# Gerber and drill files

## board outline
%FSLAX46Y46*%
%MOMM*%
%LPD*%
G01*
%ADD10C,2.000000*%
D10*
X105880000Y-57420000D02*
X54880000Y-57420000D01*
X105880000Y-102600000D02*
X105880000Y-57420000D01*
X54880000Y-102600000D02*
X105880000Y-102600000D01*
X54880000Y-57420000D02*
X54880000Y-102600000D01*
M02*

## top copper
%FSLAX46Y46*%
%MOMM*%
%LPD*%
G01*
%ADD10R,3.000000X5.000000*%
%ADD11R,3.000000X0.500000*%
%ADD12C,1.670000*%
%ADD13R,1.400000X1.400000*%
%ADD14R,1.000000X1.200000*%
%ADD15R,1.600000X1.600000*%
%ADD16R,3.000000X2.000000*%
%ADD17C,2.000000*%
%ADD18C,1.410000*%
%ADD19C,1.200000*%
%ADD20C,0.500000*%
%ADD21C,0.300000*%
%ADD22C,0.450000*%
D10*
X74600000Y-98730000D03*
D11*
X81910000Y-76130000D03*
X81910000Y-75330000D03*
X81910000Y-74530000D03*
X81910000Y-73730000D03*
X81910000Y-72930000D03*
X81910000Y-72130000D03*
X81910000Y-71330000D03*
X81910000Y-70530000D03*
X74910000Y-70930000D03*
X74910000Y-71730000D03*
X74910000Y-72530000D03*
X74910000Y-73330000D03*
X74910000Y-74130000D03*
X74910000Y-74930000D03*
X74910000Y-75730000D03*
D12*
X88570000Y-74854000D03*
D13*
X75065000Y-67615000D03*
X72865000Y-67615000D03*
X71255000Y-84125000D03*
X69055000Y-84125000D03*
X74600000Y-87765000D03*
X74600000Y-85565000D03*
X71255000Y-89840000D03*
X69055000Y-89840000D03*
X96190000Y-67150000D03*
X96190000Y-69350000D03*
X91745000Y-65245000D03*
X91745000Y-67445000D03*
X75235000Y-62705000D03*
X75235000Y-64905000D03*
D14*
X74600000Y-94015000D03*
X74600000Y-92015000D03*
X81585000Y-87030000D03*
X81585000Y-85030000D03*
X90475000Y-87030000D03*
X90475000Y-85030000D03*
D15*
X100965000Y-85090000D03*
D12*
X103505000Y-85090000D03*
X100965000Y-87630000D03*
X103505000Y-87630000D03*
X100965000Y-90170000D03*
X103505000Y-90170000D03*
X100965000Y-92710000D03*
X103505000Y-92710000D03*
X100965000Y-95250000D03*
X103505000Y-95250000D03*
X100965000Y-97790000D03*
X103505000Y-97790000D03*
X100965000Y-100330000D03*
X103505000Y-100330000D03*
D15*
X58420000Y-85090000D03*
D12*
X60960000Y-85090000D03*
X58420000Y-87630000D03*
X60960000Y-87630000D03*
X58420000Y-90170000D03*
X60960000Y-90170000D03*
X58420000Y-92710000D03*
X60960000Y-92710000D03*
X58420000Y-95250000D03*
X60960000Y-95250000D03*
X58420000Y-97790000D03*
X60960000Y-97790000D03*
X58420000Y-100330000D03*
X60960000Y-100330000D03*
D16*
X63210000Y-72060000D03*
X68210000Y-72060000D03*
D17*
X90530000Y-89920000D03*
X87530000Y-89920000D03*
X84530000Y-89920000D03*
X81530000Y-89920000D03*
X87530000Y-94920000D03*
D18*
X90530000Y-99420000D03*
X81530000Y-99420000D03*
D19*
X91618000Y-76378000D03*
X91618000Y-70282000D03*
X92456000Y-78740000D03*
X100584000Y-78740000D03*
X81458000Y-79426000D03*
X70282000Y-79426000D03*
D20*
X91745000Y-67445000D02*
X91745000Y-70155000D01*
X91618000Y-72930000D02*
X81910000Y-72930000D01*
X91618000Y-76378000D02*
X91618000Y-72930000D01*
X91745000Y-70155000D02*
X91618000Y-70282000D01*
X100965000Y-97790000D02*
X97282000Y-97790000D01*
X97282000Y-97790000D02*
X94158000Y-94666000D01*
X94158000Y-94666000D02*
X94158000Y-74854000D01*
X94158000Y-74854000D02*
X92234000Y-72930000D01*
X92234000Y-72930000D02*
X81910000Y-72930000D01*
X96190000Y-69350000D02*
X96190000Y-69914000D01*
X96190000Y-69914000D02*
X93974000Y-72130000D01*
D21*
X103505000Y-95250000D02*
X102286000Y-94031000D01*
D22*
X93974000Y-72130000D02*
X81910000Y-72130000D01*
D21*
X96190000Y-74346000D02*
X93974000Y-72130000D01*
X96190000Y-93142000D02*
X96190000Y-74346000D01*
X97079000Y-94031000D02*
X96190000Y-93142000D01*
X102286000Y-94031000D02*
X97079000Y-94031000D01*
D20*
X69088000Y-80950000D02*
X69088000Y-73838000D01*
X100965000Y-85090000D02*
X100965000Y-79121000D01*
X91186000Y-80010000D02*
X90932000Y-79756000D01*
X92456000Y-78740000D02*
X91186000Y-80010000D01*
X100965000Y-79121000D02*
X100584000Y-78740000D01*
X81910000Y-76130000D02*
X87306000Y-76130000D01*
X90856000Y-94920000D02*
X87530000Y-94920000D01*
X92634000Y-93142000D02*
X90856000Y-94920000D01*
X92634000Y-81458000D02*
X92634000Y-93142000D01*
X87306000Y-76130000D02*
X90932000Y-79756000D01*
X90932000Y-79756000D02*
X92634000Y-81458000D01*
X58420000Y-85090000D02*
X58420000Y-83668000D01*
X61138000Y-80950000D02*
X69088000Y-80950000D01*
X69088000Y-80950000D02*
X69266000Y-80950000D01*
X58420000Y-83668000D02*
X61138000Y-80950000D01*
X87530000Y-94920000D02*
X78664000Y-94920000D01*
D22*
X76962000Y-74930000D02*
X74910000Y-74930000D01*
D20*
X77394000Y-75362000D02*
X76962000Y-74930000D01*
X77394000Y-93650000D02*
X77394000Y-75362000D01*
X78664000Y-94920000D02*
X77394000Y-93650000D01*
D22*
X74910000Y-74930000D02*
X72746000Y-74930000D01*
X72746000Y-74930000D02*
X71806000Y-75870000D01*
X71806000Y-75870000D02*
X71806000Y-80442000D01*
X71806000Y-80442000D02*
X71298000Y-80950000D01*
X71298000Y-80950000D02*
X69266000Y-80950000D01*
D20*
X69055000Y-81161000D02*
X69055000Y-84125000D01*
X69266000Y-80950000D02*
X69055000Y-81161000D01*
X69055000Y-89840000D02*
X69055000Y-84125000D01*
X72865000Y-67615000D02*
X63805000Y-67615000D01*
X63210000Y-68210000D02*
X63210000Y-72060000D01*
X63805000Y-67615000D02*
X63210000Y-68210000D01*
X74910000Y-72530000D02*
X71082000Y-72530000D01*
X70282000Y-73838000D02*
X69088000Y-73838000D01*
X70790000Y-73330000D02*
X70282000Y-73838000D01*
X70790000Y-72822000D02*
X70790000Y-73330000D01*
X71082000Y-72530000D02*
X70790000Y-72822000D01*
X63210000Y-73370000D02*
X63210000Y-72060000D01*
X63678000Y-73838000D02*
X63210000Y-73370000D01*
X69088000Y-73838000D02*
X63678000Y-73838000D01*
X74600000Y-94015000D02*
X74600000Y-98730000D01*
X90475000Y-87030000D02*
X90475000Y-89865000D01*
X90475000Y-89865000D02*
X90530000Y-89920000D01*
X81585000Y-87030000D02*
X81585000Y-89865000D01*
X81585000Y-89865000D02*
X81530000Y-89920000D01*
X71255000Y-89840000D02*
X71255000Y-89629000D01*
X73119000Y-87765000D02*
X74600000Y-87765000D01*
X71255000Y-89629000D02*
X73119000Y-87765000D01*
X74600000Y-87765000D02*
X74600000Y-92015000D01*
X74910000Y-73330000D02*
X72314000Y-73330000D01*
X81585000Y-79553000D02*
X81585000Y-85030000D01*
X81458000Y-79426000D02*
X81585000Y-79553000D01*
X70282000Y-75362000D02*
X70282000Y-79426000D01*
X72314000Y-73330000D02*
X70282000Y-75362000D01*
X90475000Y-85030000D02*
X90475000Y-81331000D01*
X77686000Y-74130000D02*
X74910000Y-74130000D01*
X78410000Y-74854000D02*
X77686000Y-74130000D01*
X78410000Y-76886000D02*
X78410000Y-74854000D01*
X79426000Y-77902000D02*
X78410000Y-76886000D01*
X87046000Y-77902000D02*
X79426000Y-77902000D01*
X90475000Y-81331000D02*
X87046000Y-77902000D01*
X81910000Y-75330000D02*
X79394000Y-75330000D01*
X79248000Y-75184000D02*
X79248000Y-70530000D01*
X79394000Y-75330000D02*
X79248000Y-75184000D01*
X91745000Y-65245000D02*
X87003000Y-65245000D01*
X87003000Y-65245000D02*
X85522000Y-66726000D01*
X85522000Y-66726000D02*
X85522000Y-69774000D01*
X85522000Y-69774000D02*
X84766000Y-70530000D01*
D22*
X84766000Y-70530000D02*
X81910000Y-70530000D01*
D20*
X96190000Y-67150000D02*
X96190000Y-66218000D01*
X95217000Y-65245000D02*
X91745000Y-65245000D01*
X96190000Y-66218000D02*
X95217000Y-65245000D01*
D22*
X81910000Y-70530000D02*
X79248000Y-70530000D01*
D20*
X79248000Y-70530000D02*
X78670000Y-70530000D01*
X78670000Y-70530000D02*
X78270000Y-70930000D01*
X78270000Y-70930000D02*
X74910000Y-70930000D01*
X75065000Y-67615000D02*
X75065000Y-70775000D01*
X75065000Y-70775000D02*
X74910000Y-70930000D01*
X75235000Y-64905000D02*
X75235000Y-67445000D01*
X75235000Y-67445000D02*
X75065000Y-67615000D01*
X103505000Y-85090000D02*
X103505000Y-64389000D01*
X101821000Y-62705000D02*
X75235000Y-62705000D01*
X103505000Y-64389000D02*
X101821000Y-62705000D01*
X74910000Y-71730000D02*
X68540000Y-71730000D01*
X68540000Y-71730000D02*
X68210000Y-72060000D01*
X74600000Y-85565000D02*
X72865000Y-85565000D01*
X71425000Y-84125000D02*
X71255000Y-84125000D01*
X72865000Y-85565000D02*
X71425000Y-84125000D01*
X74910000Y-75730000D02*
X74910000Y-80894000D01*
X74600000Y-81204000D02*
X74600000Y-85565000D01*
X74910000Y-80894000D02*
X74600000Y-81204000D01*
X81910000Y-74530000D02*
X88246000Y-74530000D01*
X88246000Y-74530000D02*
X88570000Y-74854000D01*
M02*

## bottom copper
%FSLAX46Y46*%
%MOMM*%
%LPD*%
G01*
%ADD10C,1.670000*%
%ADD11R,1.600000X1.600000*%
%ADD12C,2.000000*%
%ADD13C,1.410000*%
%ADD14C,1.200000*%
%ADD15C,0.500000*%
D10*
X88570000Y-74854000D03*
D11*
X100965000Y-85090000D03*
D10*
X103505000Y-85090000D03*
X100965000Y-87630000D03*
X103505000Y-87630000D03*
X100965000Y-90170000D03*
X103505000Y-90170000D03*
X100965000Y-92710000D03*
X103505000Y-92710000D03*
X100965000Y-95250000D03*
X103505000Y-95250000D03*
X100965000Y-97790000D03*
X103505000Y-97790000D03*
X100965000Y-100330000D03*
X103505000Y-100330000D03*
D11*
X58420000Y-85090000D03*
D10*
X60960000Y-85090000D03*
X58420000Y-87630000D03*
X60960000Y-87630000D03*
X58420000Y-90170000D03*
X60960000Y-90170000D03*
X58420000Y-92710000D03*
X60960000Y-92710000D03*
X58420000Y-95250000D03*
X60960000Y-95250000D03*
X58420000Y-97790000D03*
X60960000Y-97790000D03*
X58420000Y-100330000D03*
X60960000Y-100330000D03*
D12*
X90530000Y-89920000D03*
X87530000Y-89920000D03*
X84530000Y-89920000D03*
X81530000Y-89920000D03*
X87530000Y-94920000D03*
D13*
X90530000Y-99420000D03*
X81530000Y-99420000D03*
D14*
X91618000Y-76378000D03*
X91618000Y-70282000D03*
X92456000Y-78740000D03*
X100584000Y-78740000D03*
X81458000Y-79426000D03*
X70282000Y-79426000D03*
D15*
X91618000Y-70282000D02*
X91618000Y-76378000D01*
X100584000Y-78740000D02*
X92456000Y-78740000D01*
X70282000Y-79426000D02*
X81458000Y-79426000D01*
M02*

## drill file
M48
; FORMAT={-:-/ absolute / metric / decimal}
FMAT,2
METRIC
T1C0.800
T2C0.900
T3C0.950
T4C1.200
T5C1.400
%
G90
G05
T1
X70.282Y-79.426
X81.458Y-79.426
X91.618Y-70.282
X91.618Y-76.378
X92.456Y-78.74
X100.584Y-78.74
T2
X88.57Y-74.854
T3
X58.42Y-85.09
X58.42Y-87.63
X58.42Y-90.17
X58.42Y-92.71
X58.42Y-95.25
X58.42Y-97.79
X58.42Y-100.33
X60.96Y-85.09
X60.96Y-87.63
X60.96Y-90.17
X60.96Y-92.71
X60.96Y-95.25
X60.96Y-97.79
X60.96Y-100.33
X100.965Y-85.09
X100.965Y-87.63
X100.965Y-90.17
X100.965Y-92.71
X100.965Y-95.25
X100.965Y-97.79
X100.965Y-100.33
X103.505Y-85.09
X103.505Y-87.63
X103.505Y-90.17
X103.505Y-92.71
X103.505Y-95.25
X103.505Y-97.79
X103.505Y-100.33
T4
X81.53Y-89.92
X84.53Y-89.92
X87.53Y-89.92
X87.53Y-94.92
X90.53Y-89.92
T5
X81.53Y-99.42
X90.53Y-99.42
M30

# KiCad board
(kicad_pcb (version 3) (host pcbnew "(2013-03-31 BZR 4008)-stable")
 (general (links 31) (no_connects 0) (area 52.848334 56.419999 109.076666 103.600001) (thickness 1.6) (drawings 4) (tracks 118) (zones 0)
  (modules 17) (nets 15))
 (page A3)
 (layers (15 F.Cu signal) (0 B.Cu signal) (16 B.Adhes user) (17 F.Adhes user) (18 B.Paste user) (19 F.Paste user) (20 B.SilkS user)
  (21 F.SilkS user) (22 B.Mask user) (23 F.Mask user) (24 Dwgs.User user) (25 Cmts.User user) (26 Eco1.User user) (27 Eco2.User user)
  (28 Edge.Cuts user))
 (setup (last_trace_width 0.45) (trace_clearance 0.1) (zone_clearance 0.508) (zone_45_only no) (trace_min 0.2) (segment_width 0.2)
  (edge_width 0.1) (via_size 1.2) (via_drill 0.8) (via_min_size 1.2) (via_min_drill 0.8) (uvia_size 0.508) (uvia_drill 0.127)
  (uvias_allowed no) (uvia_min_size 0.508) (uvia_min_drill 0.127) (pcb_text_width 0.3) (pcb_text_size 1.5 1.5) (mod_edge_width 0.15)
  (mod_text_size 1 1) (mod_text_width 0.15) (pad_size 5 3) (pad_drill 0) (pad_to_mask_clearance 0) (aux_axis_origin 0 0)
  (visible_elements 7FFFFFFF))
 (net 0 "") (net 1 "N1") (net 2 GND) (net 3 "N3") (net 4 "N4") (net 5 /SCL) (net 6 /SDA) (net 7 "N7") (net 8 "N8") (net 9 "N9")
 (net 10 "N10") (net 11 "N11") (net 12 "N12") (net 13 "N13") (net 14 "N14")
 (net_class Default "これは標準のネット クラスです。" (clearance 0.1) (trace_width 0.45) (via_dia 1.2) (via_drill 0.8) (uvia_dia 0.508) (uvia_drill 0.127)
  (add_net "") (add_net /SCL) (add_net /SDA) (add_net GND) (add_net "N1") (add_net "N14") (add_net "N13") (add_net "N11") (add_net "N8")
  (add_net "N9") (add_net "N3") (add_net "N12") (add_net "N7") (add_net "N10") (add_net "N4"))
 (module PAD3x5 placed (layer F.Cu) (at 74.6 98.73 90)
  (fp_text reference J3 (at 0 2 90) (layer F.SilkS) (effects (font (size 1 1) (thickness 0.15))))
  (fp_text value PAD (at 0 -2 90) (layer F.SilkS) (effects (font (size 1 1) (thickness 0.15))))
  (pad 1 smd rect (at 0 0 90) (size 5 3) (layers F.Cu F.Paste F.Mask) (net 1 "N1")))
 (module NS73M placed (layer F.Cu) (at 78.41 73.33)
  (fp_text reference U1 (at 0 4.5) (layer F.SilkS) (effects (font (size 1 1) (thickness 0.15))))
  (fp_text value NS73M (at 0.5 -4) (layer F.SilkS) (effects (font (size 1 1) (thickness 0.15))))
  (pad 1 smd rect (at 3.5 2.8) (size 3 0.5) (layers F.Cu F.Paste F.Mask) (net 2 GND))
  (pad 2 smd rect (at 3.5 2) (size 3 0.5) (layers F.Cu F.Paste F.Mask) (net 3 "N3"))
  (pad 3 smd rect (at 3.5 1.2) (size 3 0.5) (layers F.Cu F.Paste F.Mask) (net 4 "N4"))
  (pad 4 smd rect (at 3.5 0.4) (size 3 0.5) (layers F.Cu F.Paste F.Mask))
  (pad 5 smd rect (at 3.5 -0.4) (size 3 0.5) (layers F.Cu F.Paste F.Mask) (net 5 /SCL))
  (pad 6 smd rect (at 3.5 -1.2) (size 3 0.5) (layers F.Cu F.Paste F.Mask) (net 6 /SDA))
  (pad 7 smd rect (at 3.5 -2) (size 3 0.5) (layers F.Cu F.Paste F.Mask))
  (pad 8 smd rect (at 3.5 -2.8) (size 3 0.5) (layers F.Cu F.Paste F.Mask) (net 3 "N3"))
  (pad 9 smd rect (at -3.5 -2.4) (size 3 0.5) (layers F.Cu F.Paste F.Mask) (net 3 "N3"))
  (pad 10 smd rect (at -3.5 -1.6) (size 3 0.5) (layers F.Cu F.Paste F.Mask) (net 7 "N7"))
  (pad 11 smd rect (at -3.5 -0.8) (size 3 0.5) (layers F.Cu F.Paste F.Mask) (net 2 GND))
  (pad 12 smd rect (at -3.5 0) (size 3 0.5) (layers F.Cu F.Paste F.Mask) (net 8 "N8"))
  (pad 13 smd rect (at -3.5 0.8) (size 3 0.5) (layers F.Cu F.Paste F.Mask) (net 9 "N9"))
  (pad 14 smd rect (at -3.5 1.6) (size 3 0.5) (layers F.Cu F.Paste F.Mask) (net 2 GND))
  (pad 15 smd rect (at -3.5 2.4) (size 3 0.5) (layers F.Cu F.Paste F.Mask) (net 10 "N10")))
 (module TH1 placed (layer F.Cu) (at 88.57 74.854)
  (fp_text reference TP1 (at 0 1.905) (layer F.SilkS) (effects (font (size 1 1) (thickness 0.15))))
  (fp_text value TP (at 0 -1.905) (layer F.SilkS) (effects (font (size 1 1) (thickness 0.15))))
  (pad 1 thru_hole circle (at 0 0) (size 1.67 1.67) (drill 0.9) (layers *.Cu *.Mask F.SilkS) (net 4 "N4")))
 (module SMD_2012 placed (layer F.Cu) (at 73.965 67.615 180)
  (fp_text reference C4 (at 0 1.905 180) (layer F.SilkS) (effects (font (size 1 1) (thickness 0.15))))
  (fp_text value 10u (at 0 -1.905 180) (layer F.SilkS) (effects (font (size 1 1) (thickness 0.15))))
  (pad 1 smd rect (at -1.1 0 180) (size 1.4 1.4) (layers F.Cu F.Paste F.Mask) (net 3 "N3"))
  (pad 2 smd rect (at 1.1 0 180) (size 1.4 1.4) (layers F.Cu F.Paste F.Mask) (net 2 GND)))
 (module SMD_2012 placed (layer F.Cu) (at 70.155 84.125 180)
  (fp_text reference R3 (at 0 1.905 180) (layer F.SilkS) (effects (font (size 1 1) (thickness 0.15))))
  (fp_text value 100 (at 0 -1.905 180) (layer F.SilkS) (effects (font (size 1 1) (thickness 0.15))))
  (pad 1 smd rect (at -1.1 0 180) (size 1.4 1.4) (layers F.Cu F.Paste F.Mask) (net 10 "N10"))
  (pad 2 smd rect (at 1.1 0 180) (size 1.4 1.4) (layers F.Cu F.Paste F.Mask) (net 2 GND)))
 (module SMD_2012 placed (layer F.Cu) (at 74.6 86.665 90)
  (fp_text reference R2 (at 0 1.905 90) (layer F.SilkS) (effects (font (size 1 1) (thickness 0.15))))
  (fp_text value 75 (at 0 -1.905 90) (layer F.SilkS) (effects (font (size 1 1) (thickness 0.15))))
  (pad 1 smd rect (at -1.1 0 90) (size 1.4 1.4) (layers F.Cu F.Paste F.Mask) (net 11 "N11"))
  (pad 2 smd rect (at 1.1 0 90) (size 1.4 1.4) (layers F.Cu F.Paste F.Mask) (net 10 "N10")))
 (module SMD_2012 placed (layer F.Cu) (at 70.155 89.84 180)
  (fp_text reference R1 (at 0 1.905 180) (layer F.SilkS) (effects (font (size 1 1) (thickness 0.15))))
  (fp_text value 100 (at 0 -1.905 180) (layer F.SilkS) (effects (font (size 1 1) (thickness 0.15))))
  (pad 1 smd rect (at -1.1 0 180) (size 1.4 1.4) (layers F.Cu F.Paste F.Mask) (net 11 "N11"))
  (pad 2 smd rect (at 1.1 0 180) (size 1.4 1.4) (layers F.Cu F.Paste F.Mask) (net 2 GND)))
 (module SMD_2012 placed (layer F.Cu) (at 96.19 68.25 270)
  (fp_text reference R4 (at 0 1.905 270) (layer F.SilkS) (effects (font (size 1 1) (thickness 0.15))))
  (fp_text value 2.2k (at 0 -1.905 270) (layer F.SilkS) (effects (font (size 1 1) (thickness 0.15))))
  (pad 1 smd rect (at -1.1 0 270) (size 1.4 1.4) (layers F.Cu F.Paste F.Mask) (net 3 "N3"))
  (pad 2 smd rect (at 1.1 0 270) (size 1.4 1.4) (layers F.Cu F.Paste F.Mask) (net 6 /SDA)))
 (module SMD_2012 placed (layer F.Cu) (at 91.745 66.345 270)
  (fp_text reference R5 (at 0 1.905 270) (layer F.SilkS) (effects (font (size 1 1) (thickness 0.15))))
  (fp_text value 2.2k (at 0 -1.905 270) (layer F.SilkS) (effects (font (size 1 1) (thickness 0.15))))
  (pad 1 smd rect (at -1.1 0 270) (size 1.4 1.4) (layers F.Cu F.Paste F.Mask) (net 3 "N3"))
  (pad 2 smd rect (at 1.1 0 270) (size 1.4 1.4) (layers F.Cu F.Paste F.Mask) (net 5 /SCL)))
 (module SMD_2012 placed (layer F.Cu) (at 75.235 63.805 270)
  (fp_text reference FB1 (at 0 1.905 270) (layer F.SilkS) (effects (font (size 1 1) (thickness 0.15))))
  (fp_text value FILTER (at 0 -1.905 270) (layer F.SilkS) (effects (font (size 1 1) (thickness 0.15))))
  (pad 1 smd rect (at -1.1 0 270) (size 1.4 1.4) (layers F.Cu F.Paste F.Mask) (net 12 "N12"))
  (pad 2 smd rect (at 1.1 0 270) (size 1.4 1.4) (layers F.Cu F.Paste F.Mask) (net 3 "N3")))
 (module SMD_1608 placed (layer F.Cu) (at 74.6 93.015 90)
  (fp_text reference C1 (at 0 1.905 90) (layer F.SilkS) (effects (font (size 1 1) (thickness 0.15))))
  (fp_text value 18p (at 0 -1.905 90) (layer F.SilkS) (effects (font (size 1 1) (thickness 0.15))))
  (pad 1 smd rect (at -1 0 90) (size 1.2 1) (layers F.Cu F.Paste F.Mask) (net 1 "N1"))
  (pad 2 smd rect (at 1 0 90) (size 1.2 1) (layers F.Cu F.Paste F.Mask) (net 11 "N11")))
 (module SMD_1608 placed (layer F.Cu) (at 81.585 86.03 90)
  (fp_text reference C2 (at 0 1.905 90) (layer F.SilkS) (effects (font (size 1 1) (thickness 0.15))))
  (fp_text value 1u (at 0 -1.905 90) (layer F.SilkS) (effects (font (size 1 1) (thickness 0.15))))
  (pad 1 smd rect (at -1 0 90) (size 1.2 1) (layers F.Cu F.Paste F.Mask) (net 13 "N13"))
  (pad 2 smd rect (at 1 0 90) (size 1.2 1) (layers F.Cu F.Paste F.Mask) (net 8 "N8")))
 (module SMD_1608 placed (layer F.Cu) (at 90.475 86.03 90)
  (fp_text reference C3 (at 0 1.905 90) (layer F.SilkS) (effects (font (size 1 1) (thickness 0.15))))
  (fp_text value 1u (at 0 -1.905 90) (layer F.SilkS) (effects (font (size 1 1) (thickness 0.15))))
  (pad 1 smd rect (at -1 0 90) (size 1.2 1) (layers F.Cu F.Paste F.Mask) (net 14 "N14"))
  (pad 2 smd rect (at 1 0 90) (size 1.2 1) (layers F.Cu F.Paste F.Mask) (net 9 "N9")))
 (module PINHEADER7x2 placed (layer F.Cu) (at 102.235 92.71)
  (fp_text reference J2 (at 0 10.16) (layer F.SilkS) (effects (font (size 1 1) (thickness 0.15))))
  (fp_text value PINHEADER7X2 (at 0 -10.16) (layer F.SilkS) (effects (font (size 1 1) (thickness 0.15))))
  (pad 1 thru_hole rect (at -1.27 -7.62) (size 1.6 1.6) (drill 0.95) (layers *.Cu *.Mask F.SilkS) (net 2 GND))
  (pad 2 thru_hole circle (at 1.27 -7.62) (size 1.67 1.67) (drill 0.95) (layers *.Cu *.Mask F.SilkS) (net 12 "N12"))
  (pad 3 thru_hole circle (at -1.27 -5.08) (size 1.67 1.67) (drill 0.95) (layers *.Cu *.Mask F.SilkS))
  (pad 4 thru_hole circle (at 1.27 -5.08) (size 1.67 1.67) (drill 0.95) (layers *.Cu *.Mask F.SilkS))
  (pad 5 thru_hole circle (at -1.27 -2.54) (size 1.67 1.67) (drill 0.95) (layers *.Cu *.Mask F.SilkS))
  (pad 6 thru_hole circle (at 1.27 -2.54) (size 1.67 1.67) (drill 0.95) (layers *.Cu *.Mask F.SilkS))
  (pad 7 thru_hole circle (at -1.27 0) (size 1.67 1.67) (drill 0.95) (layers *.Cu *.Mask F.SilkS))
  (pad 8 thru_hole circle (at 1.27 0) (size 1.67 1.67) (drill 0.95) (layers *.Cu *.Mask F.SilkS))
  (pad 9 thru_hole circle (at -1.27 2.54) (size 1.67 1.67) (drill 0.95) (layers *.Cu *.Mask F.SilkS))
  (pad 10 thru_hole circle (at 1.27 2.54) (size 1.67 1.67) (drill 0.95) (layers *.Cu *.Mask F.SilkS) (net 6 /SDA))
  (pad 11 thru_hole circle (at -1.27 5.08) (size 1.67 1.67) (drill 0.95) (layers *.Cu *.Mask F.SilkS) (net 5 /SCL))
  (pad 12 thru_hole circle (at 1.27 5.08) (size 1.67 1.67) (drill 0.95) (layers *.Cu *.Mask F.SilkS))
  (pad 13 thru_hole circle (at -1.27 7.62) (size 1.67 1.67) (drill 0.95) (layers *.Cu *.Mask F.SilkS))
  (pad 14 thru_hole circle (at 1.27 7.62) (size 1.67 1.67) (drill 0.95) (layers *.Cu *.Mask F.SilkS)))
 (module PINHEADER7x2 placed (layer F.Cu) (at 59.69 92.71)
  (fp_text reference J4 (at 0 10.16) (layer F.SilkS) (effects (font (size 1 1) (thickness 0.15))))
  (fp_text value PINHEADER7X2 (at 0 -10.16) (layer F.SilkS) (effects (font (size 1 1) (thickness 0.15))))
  (pad 1 thru_hole rect (at -1.27 -7.62) (size 1.6 1.6) (drill 0.95) (layers *.Cu *.Mask F.SilkS) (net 2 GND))
  (pad 2 thru_hole circle (at 1.27 -7.62) (size 1.67 1.67) (drill 0.95) (layers *.Cu *.Mask F.SilkS))
  (pad 3 thru_hole circle (at -1.27 -5.08) (size 1.67 1.67) (drill 0.95) (layers *.Cu *.Mask F.SilkS))
  (pad 4 thru_hole circle (at 1.27 -5.08) (size 1.67 1.67) (drill 0.95) (layers *.Cu *.Mask F.SilkS))
  (pad 5 thru_hole circle (at -1.27 -2.54) (size 1.67 1.67) (drill 0.95) (layers *.Cu *.Mask F.SilkS))
  (pad 6 thru_hole circle (at 1.27 -2.54) (size 1.67 1.67) (drill 0.95) (layers *.Cu *.Mask F.SilkS))
  (pad 7 thru_hole circle (at -1.27 0) (size 1.67 1.67) (drill 0.95) (layers *.Cu *.Mask F.SilkS))
  (pad 8 thru_hole circle (at 1.27 0) (size 1.67 1.67) (drill 0.95) (layers *.Cu *.Mask F.SilkS))
  (pad 9 thru_hole circle (at -1.27 2.54) (size 1.67 1.67) (drill 0.95) (layers *.Cu *.Mask F.SilkS))
  (pad 10 thru_hole circle (at 1.27 2.54) (size 1.67 1.67) (drill 0.95) (layers *.Cu *.Mask F.SilkS))
  (pad 11 thru_hole circle (at -1.27 5.08) (size 1.67 1.67) (drill 0.95) (layers *.Cu *.Mask F.SilkS))
  (pad 12 thru_hole circle (at 1.27 5.08) (size 1.67 1.67) (drill 0.95) (layers *.Cu *.Mask F.SilkS))
  (pad 13 thru_hole circle (at -1.27 7.62) (size 1.67 1.67) (drill 0.95) (layers *.Cu *.Mask F.SilkS))
  (pad 14 thru_hole circle (at 1.27 7.62) (size 1.67 1.67) (drill 0.95) (layers *.Cu *.Mask F.SilkS)))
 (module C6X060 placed (layer F.Cu) (at 65.71 72.06)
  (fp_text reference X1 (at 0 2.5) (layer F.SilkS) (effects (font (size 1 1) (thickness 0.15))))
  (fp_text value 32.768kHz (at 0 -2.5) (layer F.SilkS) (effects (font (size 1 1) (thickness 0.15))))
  (pad 1 smd rect (at -2.5 0) (size 3 2) (layers F.Cu F.Paste F.Mask) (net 2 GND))
  (pad 2 smd rect (at 2.5 0) (size 3 2) (layers F.Cu F.Paste F.Mask) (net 7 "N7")))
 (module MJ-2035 (layer B.Cu) (at 86.03 94.92 180)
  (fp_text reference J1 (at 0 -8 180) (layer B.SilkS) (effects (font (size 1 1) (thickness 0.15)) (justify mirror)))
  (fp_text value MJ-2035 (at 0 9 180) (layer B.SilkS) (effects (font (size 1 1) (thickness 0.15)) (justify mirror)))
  (pad 1 thru_hole circle (at -4.5 5 180) (size 2 2) (drill 1.2) (layers *.Cu *.Mask B.SilkS) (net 14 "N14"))
  (pad 2 thru_hole circle (at -1.5 5 180) (size 2 2) (drill 1.2) (layers *.Cu *.Mask B.SilkS))
  (pad 3 thru_hole circle (at 1.5 5 180) (size 2 2) (drill 1.2) (layers *.Cu *.Mask B.SilkS))
  (pad 4 thru_hole circle (at 4.5 5 180) (size 2 2) (drill 1.2) (layers *.Cu *.Mask B.SilkS) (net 13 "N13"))
  (pad 5 thru_hole circle (at -1.5 0 180) (size 2 2) (drill 1.2) (layers *.Cu *.Mask B.SilkS) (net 2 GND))
  (pad "" thru_hole circle (at -4.5 -4.5 180) (size 1.41 1.41) (drill 1.4) (layers *.Cu *.Mask B.SilkS))
  (pad "" thru_hole circle (at 4.5 -4.5 180) (size 1.41 1.41) (drill 1.4) (layers *.Cu *.Mask B.SilkS)))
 (gr_line (start 105.88 57.42) (end 54.88 57.42) (angle 90) (layer Edge.Cuts) (width 2))
 (gr_line (start 105.88 102.6) (end 105.88 57.42) (angle 90) (layer Edge.Cuts) (width 2))
 (gr_line (start 54.88 102.6) (end 105.88 102.6) (angle 90) (layer Edge.Cuts) (width 2))
 (gr_line (start 54.88 57.42) (end 54.88 102.6) (angle 90) (layer Edge.Cuts) (width 2))
 (segment (start 91.745 67.445) (end 91.745 70.155) (width 0.5) (layer F.Cu) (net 5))
 (segment (start 91.618 72.93) (end 81.91 72.93) (width 0.5) (layer F.Cu) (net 5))
 (segment (start 91.618 76.378) (end 91.618 72.93) (width 0.5) (layer F.Cu) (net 5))
 (via (at 91.618 76.378) (size 1.2) (layers F.Cu B.Cu) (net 5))
 (segment (start 91.618 70.282) (end 91.618 76.378) (width 0.5) (layer B.Cu) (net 5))
 (via (at 91.618 70.282) (size 1.2) (layers F.Cu B.Cu) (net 5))
 (segment (start 91.745 70.155) (end 91.618 70.282) (width 0.5) (layer F.Cu) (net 5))
 (segment (start 100.965 97.79) (end 97.282 97.79) (width 0.5) (layer F.Cu) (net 5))
 (segment (start 97.282 97.79) (end 94.158 94.666) (width 0.5) (layer F.Cu) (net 5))
 (segment (start 94.158 94.666) (end 94.158 74.854) (width 0.5) (layer F.Cu) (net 5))
 (segment (start 94.158 74.854) (end 92.234 72.93) (width 0.5) (layer F.Cu) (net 5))
 (segment (start 92.234 72.93) (end 81.91 72.93) (width 0.5) (layer F.Cu) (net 5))
 (segment (start 96.19 69.35) (end 96.19 69.914) (width 0.5) (layer F.Cu) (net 6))
 (segment (start 96.19 69.914) (end 93.974 72.13) (width 0.5) (layer F.Cu) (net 6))
 (segment (start 103.505 95.25) (end 102.286 94.031) (width 0.3) (layer F.Cu) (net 6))
 (segment (start 93.974 72.13) (end 81.91 72.13) (width 0.45) (layer F.Cu) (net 6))
 (segment (start 96.19 74.346) (end 93.974 72.13) (width 0.3) (layer F.Cu) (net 6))
 (segment (start 96.19 93.142) (end 96.19 74.346) (width 0.3) (layer F.Cu) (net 6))
 (segment (start 97.079 94.031) (end 96.19 93.142) (width 0.3) (layer F.Cu) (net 6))
 (segment (start 102.286 94.031) (end 97.079 94.031) (width 0.3) (layer F.Cu) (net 6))
 (segment (start 69.088 80.95) (end 69.088 73.838) (width 0.5) (layer F.Cu) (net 2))
 (segment (start 100.965 85.09) (end 100.965 79.121) (width 0.5) (layer F.Cu) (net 2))
 (segment (start 91.186 80.01) (end 90.932 79.756) (width 0.5) (layer F.Cu) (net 2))
 (segment (start 92.456 78.74) (end 91.186 80.01) (width 0.5) (layer F.Cu) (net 2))
 (via (at 92.456 78.74) (size 1.2) (layers F.Cu B.Cu) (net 2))
 (segment (start 100.584 78.74) (end 92.456 78.74) (width 0.5) (layer B.Cu) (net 2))
 (via (at 100.584 78.74) (size 1.2) (layers F.Cu B.Cu) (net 2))
 (segment (start 100.965 79.121) (end 100.584 78.74) (width 0.5) (layer F.Cu) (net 2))
 (segment (start 81.91 76.13) (end 87.306 76.13) (width 0.5) (layer F.Cu) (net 2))
 (segment (start 90.856 94.92) (end 87.53 94.92) (width 0.5) (layer F.Cu) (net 2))
 (segment (start 92.634 93.142) (end 90.856 94.92) (width 0.5) (layer F.Cu) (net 2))
 (segment (start 92.634 81.458) (end 92.634 93.142) (width 0.5) (layer F.Cu) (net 2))
 (segment (start 87.306 76.13) (end 90.932 79.756) (width 0.5) (layer F.Cu) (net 2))
 (segment (start 90.932 79.756) (end 92.634 81.458) (width 0.5) (layer F.Cu) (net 2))
 (segment (start 58.42 85.09) (end 58.42 83.668) (width 0.5) (layer F.Cu) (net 2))
 (segment (start 61.138 80.95) (end 69.088 80.95) (width 0.5) (layer F.Cu) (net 2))
 (segment (start 69.088 80.95) (end 69.266 80.95) (width 0.5) (layer F.Cu) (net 2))
 (segment (start 58.42 83.668) (end 61.138 80.95) (width 0.5) (layer F.Cu) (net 2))
 (segment (start 87.53 94.92) (end 78.664 94.92) (width 0.5) (layer F.Cu) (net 2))
 (segment (start 76.962 74.93) (end 74.91 74.93) (width 0.45) (layer F.Cu) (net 2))
 (segment (start 77.394 75.362) (end 76.962 74.93) (width 0.5) (layer F.Cu) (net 2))
 (segment (start 77.394 93.65) (end 77.394 75.362) (width 0.5) (layer F.Cu) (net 2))
 (segment (start 78.664 94.92) (end 77.394 93.65) (width 0.5) (layer F.Cu) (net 2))
 (segment (start 74.91 74.93) (end 72.746 74.93) (width 0.45) (layer F.Cu) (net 2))
 (segment (start 72.746 74.93) (end 71.806 75.87) (width 0.45) (layer F.Cu) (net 2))
 (segment (start 71.806 75.87) (end 71.806 80.442) (width 0.45) (layer F.Cu) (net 2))
 (segment (start 71.806 80.442) (end 71.298 80.95) (width 0.45) (layer F.Cu) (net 2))
 (segment (start 71.298 80.95) (end 69.266 80.95) (width 0.45) (layer F.Cu) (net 2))
 (segment (start 69.055 81.161) (end 69.055 84.125) (width 0.5) (layer F.Cu) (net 2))
 (segment (start 69.266 80.95) (end 69.055 81.161) (width 0.5) (layer F.Cu) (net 2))
 (segment (start 69.055 89.84) (end 69.055 84.125) (width 0.5) (layer F.Cu) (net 2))
 (segment (start 72.865 67.615) (end 63.805 67.615) (width 0.5) (layer F.Cu) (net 2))
 (segment (start 63.21 68.21) (end 63.21 72.06) (width 0.5) (layer F.Cu) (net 2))
 (segment (start 63.805 67.615) (end 63.21 68.21) (width 0.5) (layer F.Cu) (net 2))
 (segment (start 74.91 72.53) (end 71.082 72.53) (width 0.5) (layer F.Cu) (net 2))
 (segment (start 70.282 73.838) (end 69.088 73.838) (width 0.5) (layer F.Cu) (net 2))
 (segment (start 70.79 73.33) (end 70.282 73.838) (width 0.5) (layer F.Cu) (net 2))
 (segment (start 70.79 72.822) (end 70.79 73.33) (width 0.5) (layer F.Cu) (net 2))
 (segment (start 71.082 72.53) (end 70.79 72.822) (width 0.5) (layer F.Cu) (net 2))
 (segment (start 63.21 73.37) (end 63.21 72.06) (width 0.5) (layer F.Cu) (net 2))
 (segment (start 63.678 73.838) (end 63.21 73.37) (width 0.5) (layer F.Cu) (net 2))
 (segment (start 69.088 73.838) (end 63.678 73.838) (width 0.5) (layer F.Cu) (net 2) (status 2))
 (segment (start 74.6 94.015) (end 74.6 98.73) (width 0.5) (layer F.Cu) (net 1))
 (segment (start 90.475 87.03) (end 90.475 89.865) (width 0.5) (layer F.Cu) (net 14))
 (segment (start 90.475 89.865) (end 90.53 89.92) (width 0.5) (layer F.Cu) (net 14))
 (segment (start 81.585 87.03) (end 81.585 89.865) (width 0.5) (layer F.Cu) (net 13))
 (segment (start 81.585 89.865) (end 81.53 89.92) (width 0.5) (layer F.Cu) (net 13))
 (segment (start 71.255 89.84) (end 71.255 89.629) (width 0.5) (layer F.Cu) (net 11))
 (segment (start 73.119 87.765) (end 74.6 87.765) (width 0.5) (layer F.Cu) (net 11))
 (segment (start 71.255 89.629) (end 73.119 87.765) (width 0.5) (layer F.Cu) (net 11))
 (segment (start 74.6 87.765) (end 74.6 92.015) (width 0.5) (layer F.Cu) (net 11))
 (segment (start 74.91 73.33) (end 72.314 73.33) (width 0.5) (layer F.Cu) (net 8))
 (segment (start 81.585 79.553) (end 81.585 85.03) (width 0.5) (layer F.Cu) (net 8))
 (segment (start 81.458 79.426) (end 81.585 79.553) (width 0.5) (layer F.Cu) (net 8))
 (via (at 81.458 79.426) (size 1.2) (layers F.Cu B.Cu) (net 8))
 (segment (start 70.282 79.426) (end 81.458 79.426) (width 0.5) (layer B.Cu) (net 8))
 (via (at 70.282 79.426) (size 1.2) (layers F.Cu B.Cu) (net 8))
 (segment (start 70.282 75.362) (end 70.282 79.426) (width 0.5) (layer F.Cu) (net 8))
 (segment (start 72.314 73.33) (end 70.282 75.362) (width 0.5) (layer F.Cu) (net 8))
 (segment (start 90.475 85.03) (end 90.475 81.331) (width 0.5) (layer F.Cu) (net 9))
 (segment (start 77.686 74.13) (end 74.91 74.13) (width 0.5) (layer F.Cu) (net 9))
 (segment (start 78.41 74.854) (end 77.686 74.13) (width 0.5) (layer F.Cu) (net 9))
 (segment (start 78.41 76.886) (end 78.41 74.854) (width 0.5) (layer F.Cu) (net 9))
 (segment (start 79.426 77.902) (end 78.41 76.886) (width 0.5) (layer F.Cu) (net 9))
 (segment (start 87.046 77.902) (end 79.426 77.902) (width 0.5) (layer F.Cu) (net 9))
 (segment (start 90.475 81.331) (end 87.046 77.902) (width 0.5) (layer F.Cu) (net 9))
 (segment (start 81.91 75.33) (end 79.394 75.33) (width 0.5) (layer F.Cu) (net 3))
 (segment (start 79.248 75.184) (end 79.248 70.53) (width 0.5) (layer F.Cu) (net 3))
 (segment (start 79.394 75.33) (end 79.248 75.184) (width 0.5) (layer F.Cu) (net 3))
 (segment (start 91.745 65.245) (end 87.003 65.245) (width 0.5) (layer F.Cu) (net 3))
 (segment (start 87.003 65.245) (end 85.522 66.726) (width 0.5) (layer F.Cu) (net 3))
 (segment (start 85.522 66.726) (end 85.522 69.774) (width 0.5) (layer F.Cu) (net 3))
 (segment (start 85.522 69.774) (end 84.766 70.53) (width 0.5) (layer F.Cu) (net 3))
 (segment (start 84.766 70.53) (end 81.91 70.53) (width 0.45) (layer F.Cu) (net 3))
 (segment (start 96.19 67.15) (end 96.19 66.218) (width 0.5) (layer F.Cu) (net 3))
 (segment (start 95.217 65.245) (end 91.745 65.245) (width 0.5) (layer F.Cu) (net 3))
 (segment (start 96.19 66.218) (end 95.217 65.245) (width 0.5) (layer F.Cu) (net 3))
 (segment (start 81.91 70.53) (end 79.248 70.53) (width 0.45) (layer F.Cu) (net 3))
 (segment (start 79.248 70.53) (end 78.67 70.53) (width 0.5) (layer F.Cu) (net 3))
 (segment (start 78.67 70.53) (end 78.27 70.93) (width 0.5) (layer F.Cu) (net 3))
 (segment (start 78.27 70.93) (end 74.91 70.93) (width 0.5) (layer F.Cu) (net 3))
 (segment (start 75.065 67.615) (end 75.065 70.775) (width 0.5) (layer F.Cu) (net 3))
 (segment (start 75.065 70.775) (end 74.91 70.93) (width 0.5) (layer F.Cu) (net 3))
 (segment (start 75.235 64.905) (end 75.235 67.445) (width 0.5) (layer F.Cu) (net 3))
 (segment (start 75.235 67.445) (end 75.065 67.615) (width 0.5) (layer F.Cu) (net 3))
 (segment (start 103.505 85.09) (end 103.505 64.389) (width 0.5) (layer F.Cu) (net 12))
 (segment (start 101.821 62.705) (end 75.235 62.705) (width 0.5) (layer F.Cu) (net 12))
 (segment (start 103.505 64.389) (end 101.821 62.705) (width 0.5) (layer F.Cu) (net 12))
 (segment (start 74.91 71.73) (end 68.54 71.73) (width 0.5) (layer F.Cu) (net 7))
 (segment (start 68.54 71.73) (end 68.21 72.06) (width 0.5) (layer F.Cu) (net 7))
 (segment (start 74.6 85.565) (end 72.865 85.565) (width 0.5) (layer F.Cu) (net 10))
 (segment (start 71.425 84.125) (end 71.255 84.125) (width 0.5) (layer F.Cu) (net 10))
 (segment (start 72.865 85.565) (end 71.425 84.125) (width 0.5) (layer F.Cu) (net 10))
 (segment (start 74.91 75.73) (end 74.91 80.894) (width 0.5) (layer F.Cu) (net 10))
 (segment (start 74.6 81.204) (end 74.6 85.565) (width 0.5) (layer F.Cu) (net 10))
 (segment (start 74.91 80.894) (end 74.6 81.204) (width 0.5) (layer F.Cu) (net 10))
 (segment (start 81.91 74.53) (end 88.246 74.53) (width 0.5) (layer F.Cu) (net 4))
 (segment (start 88.246 74.53) (end 88.57 74.854) (width 0.5) (layer F.Cu) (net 4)))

